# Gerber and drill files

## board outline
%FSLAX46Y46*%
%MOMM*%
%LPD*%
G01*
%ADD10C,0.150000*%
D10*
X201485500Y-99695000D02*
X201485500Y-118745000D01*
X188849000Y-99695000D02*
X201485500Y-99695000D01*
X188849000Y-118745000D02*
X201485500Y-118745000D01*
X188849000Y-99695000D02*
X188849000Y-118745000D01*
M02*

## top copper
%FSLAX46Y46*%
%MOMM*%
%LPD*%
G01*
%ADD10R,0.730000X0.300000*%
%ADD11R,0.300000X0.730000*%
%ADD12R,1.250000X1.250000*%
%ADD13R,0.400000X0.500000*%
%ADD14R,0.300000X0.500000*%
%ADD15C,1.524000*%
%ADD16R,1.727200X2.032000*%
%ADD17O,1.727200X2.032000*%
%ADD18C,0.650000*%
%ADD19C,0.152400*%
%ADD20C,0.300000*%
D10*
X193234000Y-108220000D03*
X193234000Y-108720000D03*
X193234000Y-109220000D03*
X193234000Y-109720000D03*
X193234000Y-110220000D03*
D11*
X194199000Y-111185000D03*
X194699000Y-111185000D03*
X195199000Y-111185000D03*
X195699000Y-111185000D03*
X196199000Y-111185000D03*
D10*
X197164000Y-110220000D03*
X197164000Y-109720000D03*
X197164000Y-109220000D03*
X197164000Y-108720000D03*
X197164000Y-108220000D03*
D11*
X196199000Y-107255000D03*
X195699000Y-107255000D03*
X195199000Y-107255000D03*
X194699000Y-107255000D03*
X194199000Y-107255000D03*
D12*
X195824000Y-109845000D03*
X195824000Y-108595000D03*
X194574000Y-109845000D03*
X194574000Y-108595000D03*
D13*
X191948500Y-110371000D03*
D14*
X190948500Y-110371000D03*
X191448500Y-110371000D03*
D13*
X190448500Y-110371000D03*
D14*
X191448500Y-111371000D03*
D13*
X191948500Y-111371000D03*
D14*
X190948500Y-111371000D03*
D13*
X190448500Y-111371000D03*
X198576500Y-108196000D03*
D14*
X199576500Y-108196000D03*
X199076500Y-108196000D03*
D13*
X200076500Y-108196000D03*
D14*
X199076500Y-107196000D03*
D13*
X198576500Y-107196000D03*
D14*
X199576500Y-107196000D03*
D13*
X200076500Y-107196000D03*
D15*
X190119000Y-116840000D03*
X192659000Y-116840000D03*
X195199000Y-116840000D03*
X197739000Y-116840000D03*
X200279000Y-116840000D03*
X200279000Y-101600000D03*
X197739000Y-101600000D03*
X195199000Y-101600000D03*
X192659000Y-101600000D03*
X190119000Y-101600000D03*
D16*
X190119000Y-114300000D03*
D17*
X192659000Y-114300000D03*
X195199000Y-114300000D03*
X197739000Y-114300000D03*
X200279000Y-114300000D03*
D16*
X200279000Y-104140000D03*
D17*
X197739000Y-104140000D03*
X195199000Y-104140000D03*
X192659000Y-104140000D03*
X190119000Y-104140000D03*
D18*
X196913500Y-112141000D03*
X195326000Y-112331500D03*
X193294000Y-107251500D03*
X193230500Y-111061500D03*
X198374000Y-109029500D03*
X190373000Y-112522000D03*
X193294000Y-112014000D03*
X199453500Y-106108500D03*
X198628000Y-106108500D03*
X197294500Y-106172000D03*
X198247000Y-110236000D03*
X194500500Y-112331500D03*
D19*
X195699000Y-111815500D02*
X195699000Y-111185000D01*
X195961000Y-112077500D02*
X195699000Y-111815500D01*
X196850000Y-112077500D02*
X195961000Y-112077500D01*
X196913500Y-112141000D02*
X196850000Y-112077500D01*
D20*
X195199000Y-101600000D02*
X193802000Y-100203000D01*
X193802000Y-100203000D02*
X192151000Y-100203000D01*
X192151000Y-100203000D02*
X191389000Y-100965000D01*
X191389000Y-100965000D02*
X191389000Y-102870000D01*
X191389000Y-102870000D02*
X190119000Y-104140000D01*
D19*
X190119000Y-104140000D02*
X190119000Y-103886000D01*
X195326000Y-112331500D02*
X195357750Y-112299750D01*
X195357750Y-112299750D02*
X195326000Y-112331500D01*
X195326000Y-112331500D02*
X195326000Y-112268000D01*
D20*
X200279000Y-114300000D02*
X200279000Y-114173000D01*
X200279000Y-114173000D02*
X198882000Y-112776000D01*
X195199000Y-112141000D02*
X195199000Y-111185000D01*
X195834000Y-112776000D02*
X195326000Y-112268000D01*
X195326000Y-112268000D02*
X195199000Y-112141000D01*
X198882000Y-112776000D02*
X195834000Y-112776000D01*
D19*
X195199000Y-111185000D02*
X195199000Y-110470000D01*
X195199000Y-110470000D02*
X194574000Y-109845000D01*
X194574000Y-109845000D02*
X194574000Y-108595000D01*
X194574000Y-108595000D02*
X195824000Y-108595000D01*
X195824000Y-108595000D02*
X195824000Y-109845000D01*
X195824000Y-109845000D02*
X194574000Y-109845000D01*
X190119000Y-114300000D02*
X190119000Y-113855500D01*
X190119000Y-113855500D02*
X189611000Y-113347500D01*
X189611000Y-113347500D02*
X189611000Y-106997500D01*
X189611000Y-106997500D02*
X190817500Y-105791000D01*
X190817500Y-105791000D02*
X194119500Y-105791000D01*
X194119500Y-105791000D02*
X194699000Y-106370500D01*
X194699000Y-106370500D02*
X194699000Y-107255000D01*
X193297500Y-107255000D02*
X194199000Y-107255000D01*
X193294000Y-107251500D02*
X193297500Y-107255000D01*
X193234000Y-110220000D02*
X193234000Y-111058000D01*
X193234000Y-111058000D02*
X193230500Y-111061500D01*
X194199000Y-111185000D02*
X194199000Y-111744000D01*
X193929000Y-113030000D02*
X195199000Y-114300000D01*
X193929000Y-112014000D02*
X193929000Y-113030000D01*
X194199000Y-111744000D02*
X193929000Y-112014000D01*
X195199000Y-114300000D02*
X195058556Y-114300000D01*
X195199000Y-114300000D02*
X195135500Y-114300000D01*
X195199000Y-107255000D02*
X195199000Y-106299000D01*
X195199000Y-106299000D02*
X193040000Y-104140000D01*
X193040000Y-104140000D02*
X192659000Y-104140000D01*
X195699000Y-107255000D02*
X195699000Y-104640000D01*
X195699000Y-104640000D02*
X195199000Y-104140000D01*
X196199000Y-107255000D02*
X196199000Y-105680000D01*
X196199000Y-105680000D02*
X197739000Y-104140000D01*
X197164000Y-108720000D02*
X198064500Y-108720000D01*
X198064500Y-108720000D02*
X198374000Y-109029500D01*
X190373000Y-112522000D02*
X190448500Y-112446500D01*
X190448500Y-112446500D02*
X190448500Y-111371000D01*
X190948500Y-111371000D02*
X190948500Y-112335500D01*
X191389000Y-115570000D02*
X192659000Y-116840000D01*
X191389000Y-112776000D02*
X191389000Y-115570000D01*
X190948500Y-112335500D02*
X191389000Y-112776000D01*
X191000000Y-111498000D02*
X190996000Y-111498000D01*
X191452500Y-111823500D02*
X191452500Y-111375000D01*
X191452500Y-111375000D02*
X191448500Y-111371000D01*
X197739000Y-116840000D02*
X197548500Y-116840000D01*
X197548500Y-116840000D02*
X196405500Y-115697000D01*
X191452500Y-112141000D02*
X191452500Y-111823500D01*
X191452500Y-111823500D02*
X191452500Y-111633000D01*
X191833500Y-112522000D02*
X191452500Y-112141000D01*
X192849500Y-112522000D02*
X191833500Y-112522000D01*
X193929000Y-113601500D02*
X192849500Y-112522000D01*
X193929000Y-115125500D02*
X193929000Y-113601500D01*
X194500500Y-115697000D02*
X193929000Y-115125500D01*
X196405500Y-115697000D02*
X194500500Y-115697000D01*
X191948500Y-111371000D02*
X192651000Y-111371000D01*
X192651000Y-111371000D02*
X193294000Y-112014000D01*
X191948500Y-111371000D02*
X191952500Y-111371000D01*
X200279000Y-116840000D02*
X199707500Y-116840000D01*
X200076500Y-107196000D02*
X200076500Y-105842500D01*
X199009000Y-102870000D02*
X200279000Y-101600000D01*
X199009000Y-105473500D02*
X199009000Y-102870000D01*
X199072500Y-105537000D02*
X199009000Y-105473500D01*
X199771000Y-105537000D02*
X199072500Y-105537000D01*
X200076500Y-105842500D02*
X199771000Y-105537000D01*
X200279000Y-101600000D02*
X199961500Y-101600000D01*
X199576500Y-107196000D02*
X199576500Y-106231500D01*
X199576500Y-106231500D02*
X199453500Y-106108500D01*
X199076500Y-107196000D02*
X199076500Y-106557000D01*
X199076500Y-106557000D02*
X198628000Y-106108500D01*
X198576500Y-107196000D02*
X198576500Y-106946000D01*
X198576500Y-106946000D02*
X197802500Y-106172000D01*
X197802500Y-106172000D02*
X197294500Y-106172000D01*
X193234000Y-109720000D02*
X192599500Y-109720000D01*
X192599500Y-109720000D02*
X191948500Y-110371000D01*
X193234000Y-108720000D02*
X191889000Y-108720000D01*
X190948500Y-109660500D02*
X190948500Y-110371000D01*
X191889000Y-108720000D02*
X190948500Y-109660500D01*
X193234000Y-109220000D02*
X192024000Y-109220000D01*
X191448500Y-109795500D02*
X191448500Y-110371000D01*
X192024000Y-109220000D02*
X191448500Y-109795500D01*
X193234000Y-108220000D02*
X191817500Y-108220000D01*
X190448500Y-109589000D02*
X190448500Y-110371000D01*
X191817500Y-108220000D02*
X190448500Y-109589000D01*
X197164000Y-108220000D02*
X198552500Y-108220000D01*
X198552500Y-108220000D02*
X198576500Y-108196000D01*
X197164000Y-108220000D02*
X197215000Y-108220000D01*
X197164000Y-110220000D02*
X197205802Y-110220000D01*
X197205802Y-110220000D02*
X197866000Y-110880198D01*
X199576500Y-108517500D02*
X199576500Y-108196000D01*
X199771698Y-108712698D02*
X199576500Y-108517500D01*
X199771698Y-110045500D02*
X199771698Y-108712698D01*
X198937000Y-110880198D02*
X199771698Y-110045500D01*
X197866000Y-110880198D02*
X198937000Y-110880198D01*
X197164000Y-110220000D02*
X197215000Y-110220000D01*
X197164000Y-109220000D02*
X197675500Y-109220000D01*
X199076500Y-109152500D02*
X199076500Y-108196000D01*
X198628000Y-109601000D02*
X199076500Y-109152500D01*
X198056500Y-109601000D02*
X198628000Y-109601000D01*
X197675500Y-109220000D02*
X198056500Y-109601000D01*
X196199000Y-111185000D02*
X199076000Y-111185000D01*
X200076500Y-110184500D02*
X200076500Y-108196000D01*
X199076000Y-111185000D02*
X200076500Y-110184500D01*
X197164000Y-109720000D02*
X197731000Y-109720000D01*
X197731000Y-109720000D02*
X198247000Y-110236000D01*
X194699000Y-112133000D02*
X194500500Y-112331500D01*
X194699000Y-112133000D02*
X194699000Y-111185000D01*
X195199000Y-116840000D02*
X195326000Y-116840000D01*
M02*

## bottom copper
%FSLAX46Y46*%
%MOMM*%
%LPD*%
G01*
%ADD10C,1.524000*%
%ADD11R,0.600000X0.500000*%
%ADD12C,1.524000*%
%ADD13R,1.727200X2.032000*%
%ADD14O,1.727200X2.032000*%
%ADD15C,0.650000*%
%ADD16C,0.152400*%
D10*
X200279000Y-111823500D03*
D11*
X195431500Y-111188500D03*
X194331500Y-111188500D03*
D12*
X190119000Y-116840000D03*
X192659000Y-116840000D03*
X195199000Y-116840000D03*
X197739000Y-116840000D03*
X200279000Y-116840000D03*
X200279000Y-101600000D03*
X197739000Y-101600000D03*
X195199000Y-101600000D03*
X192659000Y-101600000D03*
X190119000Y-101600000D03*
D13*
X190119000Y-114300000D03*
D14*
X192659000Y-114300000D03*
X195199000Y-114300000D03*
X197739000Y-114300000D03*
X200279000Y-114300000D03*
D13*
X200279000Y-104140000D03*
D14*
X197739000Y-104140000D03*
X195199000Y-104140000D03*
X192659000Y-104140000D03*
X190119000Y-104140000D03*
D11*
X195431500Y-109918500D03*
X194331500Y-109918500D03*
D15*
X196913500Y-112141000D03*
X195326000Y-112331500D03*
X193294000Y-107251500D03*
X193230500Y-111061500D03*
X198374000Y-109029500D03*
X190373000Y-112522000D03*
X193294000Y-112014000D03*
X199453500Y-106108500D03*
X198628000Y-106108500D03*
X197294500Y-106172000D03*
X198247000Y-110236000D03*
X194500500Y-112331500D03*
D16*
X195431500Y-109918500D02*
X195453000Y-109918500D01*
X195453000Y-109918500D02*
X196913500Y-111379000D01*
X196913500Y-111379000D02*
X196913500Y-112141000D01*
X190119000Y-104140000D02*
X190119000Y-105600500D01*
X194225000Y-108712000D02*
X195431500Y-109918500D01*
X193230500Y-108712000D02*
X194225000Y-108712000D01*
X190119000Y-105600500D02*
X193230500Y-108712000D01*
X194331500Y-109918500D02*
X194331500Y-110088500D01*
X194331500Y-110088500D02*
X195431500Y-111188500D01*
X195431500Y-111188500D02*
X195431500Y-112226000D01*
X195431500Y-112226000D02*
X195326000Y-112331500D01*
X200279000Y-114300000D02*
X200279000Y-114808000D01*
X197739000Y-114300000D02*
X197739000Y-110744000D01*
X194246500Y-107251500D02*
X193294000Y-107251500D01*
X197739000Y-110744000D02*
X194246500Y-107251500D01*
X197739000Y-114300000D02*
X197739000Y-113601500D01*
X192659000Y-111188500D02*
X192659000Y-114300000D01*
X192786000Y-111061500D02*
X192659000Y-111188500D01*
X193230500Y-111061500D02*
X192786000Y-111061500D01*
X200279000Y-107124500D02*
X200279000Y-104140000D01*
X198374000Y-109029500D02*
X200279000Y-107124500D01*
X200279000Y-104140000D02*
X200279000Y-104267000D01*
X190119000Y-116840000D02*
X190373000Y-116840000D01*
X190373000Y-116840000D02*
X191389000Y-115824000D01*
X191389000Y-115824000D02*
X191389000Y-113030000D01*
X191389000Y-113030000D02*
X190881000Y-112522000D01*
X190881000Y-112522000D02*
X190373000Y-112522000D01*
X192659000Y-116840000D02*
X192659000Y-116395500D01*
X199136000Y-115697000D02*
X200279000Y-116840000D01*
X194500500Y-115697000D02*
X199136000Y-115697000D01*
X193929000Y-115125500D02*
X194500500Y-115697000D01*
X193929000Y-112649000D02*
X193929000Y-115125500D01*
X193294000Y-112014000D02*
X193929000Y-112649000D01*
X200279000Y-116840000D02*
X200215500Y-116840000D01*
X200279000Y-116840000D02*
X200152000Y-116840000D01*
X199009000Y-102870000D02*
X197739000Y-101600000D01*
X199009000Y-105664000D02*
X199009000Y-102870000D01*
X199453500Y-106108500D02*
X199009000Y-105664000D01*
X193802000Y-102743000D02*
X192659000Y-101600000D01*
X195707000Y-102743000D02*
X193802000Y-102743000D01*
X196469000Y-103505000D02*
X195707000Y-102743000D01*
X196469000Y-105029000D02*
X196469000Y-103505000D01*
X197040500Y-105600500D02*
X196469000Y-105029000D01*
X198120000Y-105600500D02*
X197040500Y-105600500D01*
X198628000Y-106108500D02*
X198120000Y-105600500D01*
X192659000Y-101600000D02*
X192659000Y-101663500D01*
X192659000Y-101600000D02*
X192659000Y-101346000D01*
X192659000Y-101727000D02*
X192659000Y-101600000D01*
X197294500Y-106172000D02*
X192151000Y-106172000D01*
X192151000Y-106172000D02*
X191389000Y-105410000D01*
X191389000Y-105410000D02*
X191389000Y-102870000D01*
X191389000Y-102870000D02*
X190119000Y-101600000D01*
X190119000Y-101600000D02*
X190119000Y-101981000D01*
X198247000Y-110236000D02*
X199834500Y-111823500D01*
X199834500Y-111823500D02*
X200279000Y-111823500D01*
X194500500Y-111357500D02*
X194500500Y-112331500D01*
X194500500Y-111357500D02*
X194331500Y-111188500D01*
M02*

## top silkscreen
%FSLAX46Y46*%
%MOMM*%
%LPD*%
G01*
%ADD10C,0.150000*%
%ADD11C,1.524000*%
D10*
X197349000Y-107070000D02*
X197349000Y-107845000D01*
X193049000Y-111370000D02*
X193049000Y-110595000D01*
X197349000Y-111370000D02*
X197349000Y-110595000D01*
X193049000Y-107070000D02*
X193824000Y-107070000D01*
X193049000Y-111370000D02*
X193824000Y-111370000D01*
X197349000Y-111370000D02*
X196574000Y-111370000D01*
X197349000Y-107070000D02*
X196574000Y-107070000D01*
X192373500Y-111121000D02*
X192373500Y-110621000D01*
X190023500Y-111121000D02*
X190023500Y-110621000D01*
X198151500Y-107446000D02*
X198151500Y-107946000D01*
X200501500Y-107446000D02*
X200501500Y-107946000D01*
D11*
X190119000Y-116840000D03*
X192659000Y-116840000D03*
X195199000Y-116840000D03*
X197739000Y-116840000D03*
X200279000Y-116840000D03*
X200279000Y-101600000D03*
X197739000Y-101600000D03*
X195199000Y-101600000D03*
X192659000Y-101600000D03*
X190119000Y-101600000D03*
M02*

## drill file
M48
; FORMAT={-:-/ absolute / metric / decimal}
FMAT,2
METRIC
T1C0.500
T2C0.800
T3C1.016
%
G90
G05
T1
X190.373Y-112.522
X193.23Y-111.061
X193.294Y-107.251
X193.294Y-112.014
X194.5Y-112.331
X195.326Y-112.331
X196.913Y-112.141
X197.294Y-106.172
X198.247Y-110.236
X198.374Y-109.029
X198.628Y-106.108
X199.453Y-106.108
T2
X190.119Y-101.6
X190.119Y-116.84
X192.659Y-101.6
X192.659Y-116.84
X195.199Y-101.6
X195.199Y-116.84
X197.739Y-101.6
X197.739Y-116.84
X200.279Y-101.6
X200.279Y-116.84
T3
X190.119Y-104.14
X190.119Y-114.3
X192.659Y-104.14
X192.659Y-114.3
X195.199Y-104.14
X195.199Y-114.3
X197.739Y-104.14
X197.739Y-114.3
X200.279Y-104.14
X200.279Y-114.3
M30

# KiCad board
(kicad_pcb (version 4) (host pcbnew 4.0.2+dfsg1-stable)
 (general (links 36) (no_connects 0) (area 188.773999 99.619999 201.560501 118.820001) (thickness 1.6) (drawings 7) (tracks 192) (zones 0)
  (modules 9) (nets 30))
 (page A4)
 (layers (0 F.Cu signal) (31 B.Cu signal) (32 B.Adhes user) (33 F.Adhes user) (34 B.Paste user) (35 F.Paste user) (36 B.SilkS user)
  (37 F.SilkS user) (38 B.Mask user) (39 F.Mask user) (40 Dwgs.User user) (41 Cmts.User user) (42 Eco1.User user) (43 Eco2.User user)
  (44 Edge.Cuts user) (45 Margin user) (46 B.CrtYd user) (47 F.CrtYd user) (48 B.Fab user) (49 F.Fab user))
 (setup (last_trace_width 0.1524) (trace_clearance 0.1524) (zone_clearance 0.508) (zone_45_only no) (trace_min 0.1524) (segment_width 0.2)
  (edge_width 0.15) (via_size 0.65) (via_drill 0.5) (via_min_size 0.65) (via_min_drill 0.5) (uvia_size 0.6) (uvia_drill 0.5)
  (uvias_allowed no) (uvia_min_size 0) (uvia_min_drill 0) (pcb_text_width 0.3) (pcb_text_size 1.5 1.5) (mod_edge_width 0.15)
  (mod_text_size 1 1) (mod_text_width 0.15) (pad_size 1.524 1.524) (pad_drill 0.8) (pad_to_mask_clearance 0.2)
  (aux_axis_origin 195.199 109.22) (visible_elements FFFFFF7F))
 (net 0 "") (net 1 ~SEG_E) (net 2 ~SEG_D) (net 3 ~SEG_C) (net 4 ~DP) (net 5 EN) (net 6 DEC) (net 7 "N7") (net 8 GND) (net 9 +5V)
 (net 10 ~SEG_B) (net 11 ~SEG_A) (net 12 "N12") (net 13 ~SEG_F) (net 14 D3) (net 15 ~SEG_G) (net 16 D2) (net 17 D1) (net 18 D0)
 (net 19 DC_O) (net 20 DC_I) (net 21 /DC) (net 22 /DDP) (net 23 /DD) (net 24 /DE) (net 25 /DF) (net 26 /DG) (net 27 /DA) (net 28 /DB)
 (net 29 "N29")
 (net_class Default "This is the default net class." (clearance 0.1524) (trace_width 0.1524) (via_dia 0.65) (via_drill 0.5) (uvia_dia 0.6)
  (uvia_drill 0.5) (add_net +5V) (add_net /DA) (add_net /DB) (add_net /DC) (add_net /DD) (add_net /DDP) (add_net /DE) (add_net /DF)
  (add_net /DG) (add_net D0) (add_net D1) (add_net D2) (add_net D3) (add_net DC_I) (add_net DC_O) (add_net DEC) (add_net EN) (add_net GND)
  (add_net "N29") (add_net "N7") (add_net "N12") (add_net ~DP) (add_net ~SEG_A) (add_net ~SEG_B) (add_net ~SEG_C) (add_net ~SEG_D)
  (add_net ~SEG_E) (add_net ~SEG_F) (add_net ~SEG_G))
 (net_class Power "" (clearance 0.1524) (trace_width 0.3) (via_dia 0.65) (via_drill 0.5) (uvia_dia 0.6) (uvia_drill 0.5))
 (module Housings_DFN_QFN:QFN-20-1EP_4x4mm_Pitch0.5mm (layer F.Cu) (at 195.199 109.22)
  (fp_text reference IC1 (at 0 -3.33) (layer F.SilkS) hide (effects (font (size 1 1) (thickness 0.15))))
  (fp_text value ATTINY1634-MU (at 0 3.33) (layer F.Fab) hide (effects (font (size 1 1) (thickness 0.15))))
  (fp_line (start 2.15 -2.15) (end 2.15 -1.375) (layer F.SilkS) (width 0.15))
  (fp_line (start -2.15 2.15) (end -2.15 1.375) (layer F.SilkS) (width 0.15))
  (fp_line (start 2.15 2.15) (end 2.15 1.375) (layer F.SilkS) (width 0.15))
  (fp_line (start -2.15 -2.15) (end -1.375 -2.15) (layer F.SilkS) (width 0.15))
  (fp_line (start -2.15 2.15) (end -1.375 2.15) (layer F.SilkS) (width 0.15))
  (fp_line (start 2.15 2.15) (end 1.375 2.15) (layer F.SilkS) (width 0.15))
  (fp_line (start 2.15 -2.15) (end 1.375 -2.15) (layer F.SilkS) (width 0.15))
  (pad 1 smd rect (at -1.965 -1) (size 0.73 0.3) (layers F.Cu F.Paste F.Mask) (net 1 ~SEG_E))
  (pad 2 smd rect (at -1.965 -0.5) (size 0.73 0.3) (layers F.Cu F.Paste F.Mask) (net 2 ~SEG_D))
  (pad 3 smd rect (at -1.965 0) (size 0.73 0.3) (layers F.Cu F.Paste F.Mask) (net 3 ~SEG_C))
  (pad 4 smd rect (at -1.965 0.5) (size 0.73 0.3) (layers F.Cu F.Paste F.Mask) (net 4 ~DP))
  (pad 5 smd rect (at -1.965 1) (size 0.73 0.3) (layers F.Cu F.Paste F.Mask) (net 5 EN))
  (pad 6 smd rect (at -1 1.965 90) (size 0.73 0.3) (layers F.Cu F.Paste F.Mask) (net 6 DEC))
  (pad 7 smd rect (at -0.5 1.965 90) (size 0.73 0.3) (layers F.Cu F.Paste F.Mask) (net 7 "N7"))
  (pad 8 smd rect (at 0 1.965 90) (size 0.73 0.3) (layers F.Cu F.Paste F.Mask) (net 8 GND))
  (pad 9 smd rect (at 0.5 1.965 90) (size 0.73 0.3) (layers F.Cu F.Paste F.Mask) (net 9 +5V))
  (pad 10 smd rect (at 1 1.965 90) (size 0.73 0.3) (layers F.Cu F.Paste F.Mask) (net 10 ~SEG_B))
  (pad 11 smd rect (at 1.965 1) (size 0.73 0.3) (layers F.Cu F.Paste F.Mask) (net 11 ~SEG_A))
  (pad 12 smd rect (at 1.965 0.5) (size 0.73 0.3) (layers F.Cu F.Paste F.Mask) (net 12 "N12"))
  (pad 13 smd rect (at 1.965 0) (size 0.73 0.3) (layers F.Cu F.Paste F.Mask) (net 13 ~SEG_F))
  (pad 14 smd rect (at 1.965 -0.5) (size 0.73 0.3) (layers F.Cu F.Paste F.Mask) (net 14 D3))
  (pad 15 smd rect (at 1.965 -1) (size 0.73 0.3) (layers F.Cu F.Paste F.Mask) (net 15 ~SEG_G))
  (pad 16 smd rect (at 1 -1.965 90) (size 0.73 0.3) (layers F.Cu F.Paste F.Mask) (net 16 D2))
  (pad 17 smd rect (at 0.5 -1.965 90) (size 0.73 0.3) (layers F.Cu F.Paste F.Mask) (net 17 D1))
  (pad 18 smd rect (at 0 -1.965 90) (size 0.73 0.3) (layers F.Cu F.Paste F.Mask) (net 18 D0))
  (pad 19 smd rect (at -0.5 -1.965 90) (size 0.73 0.3) (layers F.Cu F.Paste F.Mask) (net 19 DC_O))
  (pad 20 smd rect (at -1 -1.965 90) (size 0.73 0.3) (layers F.Cu F.Paste F.Mask) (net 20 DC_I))
  (pad 21 smd rect (at 0.625 0.625) (size 1.25 1.25) (layers F.Cu F.Paste F.Mask) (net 8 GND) (solder_paste_margin_ratio -0.2))
  (pad 21 smd rect (at 0.625 -0.625) (size 1.25 1.25) (layers F.Cu F.Paste F.Mask) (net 8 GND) (solder_paste_margin_ratio -0.2))
  (pad 21 smd rect (at -0.625 0.625) (size 1.25 1.25) (layers F.Cu F.Paste F.Mask) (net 8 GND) (solder_paste_margin_ratio -0.2))
  (pad 21 smd rect (at -0.625 -0.625) (size 1.25 1.25) (layers F.Cu F.Paste F.Mask) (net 8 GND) (solder_paste_margin_ratio -0.2)))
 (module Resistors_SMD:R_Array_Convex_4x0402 (layer F.Cu) (at 191.1985 110.871 270)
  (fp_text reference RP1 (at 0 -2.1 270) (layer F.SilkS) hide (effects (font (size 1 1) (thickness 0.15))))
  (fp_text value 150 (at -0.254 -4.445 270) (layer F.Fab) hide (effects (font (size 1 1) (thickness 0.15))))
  (fp_line (start 0.25 -1.175) (end -0.25 -1.175) (layer F.SilkS) (width 0.15))
  (fp_line (start 0.25 1.175) (end -0.25 1.175) (layer F.SilkS) (width 0.15))
  (pad 1 smd rect (at -0.5 -0.75 270) (size 0.5 0.4) (layers F.Cu F.Paste F.Mask) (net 4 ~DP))
  (pad 3 smd rect (at -0.5 0.25 270) (size 0.5 0.3) (layers F.Cu F.Paste F.Mask) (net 2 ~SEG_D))
  (pad 2 smd rect (at -0.5 -0.25 270) (size 0.5 0.3) (layers F.Cu F.Paste F.Mask) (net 3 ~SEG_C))
  (pad 4 smd rect (at -0.5 0.75 270) (size 0.5 0.4) (layers F.Cu F.Paste F.Mask) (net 1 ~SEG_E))
  (pad 7 smd rect (at 0.5 -0.25 270) (size 0.5 0.3) (layers F.Cu F.Paste F.Mask) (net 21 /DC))
  (pad 8 smd rect (at 0.5 -0.75 270) (size 0.5 0.4) (layers F.Cu F.Paste F.Mask) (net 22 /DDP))
  (pad 6 smd rect (at 0.5 0.25 270) (size 0.5 0.3) (layers F.Cu F.Paste F.Mask) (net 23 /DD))
  (pad 5 smd rect (at 0.5 0.75 270) (size 0.5 0.4) (layers F.Cu F.Paste F.Mask) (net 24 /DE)))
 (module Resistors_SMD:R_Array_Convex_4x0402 (layer F.Cu) (at 199.3265 107.696 90)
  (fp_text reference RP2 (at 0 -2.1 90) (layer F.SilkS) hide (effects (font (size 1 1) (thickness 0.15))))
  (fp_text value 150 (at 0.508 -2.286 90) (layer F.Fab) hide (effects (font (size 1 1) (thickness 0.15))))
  (fp_line (start 0.25 -1.175) (end -0.25 -1.175) (layer F.SilkS) (width 0.15))
  (fp_line (start 0.25 1.175) (end -0.25 1.175) (layer F.SilkS) (width 0.15))
  (pad 1 smd rect (at -0.5 -0.75 90) (size 0.5 0.4) (layers F.Cu F.Paste F.Mask) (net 15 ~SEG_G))
  (pad 3 smd rect (at -0.5 0.25 90) (size 0.5 0.3) (layers F.Cu F.Paste F.Mask) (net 11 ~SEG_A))
  (pad 2 smd rect (at -0.5 -0.25 90) (size 0.5 0.3) (layers F.Cu F.Paste F.Mask) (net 13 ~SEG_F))
  (pad 4 smd rect (at -0.5 0.75 90) (size 0.5 0.4) (layers F.Cu F.Paste F.Mask) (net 10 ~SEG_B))
  (pad 7 smd rect (at 0.5 -0.25 90) (size 0.5 0.3) (layers F.Cu F.Paste F.Mask) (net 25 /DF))
  (pad 8 smd rect (at 0.5 -0.75 90) (size 0.5 0.4) (layers F.Cu F.Paste F.Mask) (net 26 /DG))
  (pad 6 smd rect (at 0.5 0.25 90) (size 0.5 0.3) (layers F.Cu F.Paste F.Mask) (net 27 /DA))
  (pad 5 smd rect (at 0.5 0.75 90) (size 0.5 0.4) (layers F.Cu F.Paste F.Mask) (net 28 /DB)))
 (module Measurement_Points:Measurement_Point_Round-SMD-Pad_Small (layer B.Cu) (at 200.279 111.8235)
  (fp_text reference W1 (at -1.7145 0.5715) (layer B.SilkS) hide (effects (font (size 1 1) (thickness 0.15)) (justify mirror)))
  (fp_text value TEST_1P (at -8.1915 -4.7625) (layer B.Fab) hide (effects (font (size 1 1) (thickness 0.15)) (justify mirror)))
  (pad 1 smd circle (at 0 0) (size 1.524 1.524) (layers B.Cu B.Paste B.Mask) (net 12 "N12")))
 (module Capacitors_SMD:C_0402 (layer B.Cu) (at 194.8815 111.1885 180)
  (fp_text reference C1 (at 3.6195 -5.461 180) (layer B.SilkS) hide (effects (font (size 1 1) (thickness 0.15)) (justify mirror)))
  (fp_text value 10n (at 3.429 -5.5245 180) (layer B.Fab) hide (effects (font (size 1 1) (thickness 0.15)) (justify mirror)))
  (pad 1 smd rect (at -0.55 0 180) (size 0.6 0.5) (layers B.Cu B.Paste B.Mask) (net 8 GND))
  (pad 2 smd rect (at 0.55 0 180) (size 0.6 0.5) (layers B.Cu B.Paste B.Mask) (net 7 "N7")))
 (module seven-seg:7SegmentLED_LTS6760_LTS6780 (layer F.Cu) (at 195.199 109.22)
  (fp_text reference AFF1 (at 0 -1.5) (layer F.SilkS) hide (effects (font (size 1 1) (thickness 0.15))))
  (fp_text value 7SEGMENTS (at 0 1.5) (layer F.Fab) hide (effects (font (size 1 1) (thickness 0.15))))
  (pad 1 thru_hole circle (at -5.08 7.62) (size 1.524 1.524) (drill 0.8) (layers *.Cu *.Mask F.SilkS) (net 24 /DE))
  (pad 2 thru_hole circle (at -2.54 7.62) (size 1.524 1.524) (drill 0.8) (layers *.Cu *.Mask F.SilkS) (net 23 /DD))
  (pad 3 thru_hole circle (at 0 7.62) (size 1.524 1.524) (drill 0.8) (layers *.Cu *.Mask F.SilkS) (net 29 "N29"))
  (pad 4 thru_hole circle (at 2.54 7.62) (size 1.524 1.524) (drill 0.8) (layers *.Cu *.Mask F.SilkS) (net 21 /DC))
  (pad 5 thru_hole circle (at 5.08 7.62) (size 1.524 1.524) (drill 0.8) (layers *.Cu *.Mask F.SilkS) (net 22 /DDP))
  (pad 6 thru_hole circle (at 5.08 -7.62) (size 1.524 1.524) (drill 0.8) (layers *.Cu *.Mask F.SilkS) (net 28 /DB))
  (pad 7 thru_hole circle (at 2.54 -7.62) (size 1.524 1.524) (drill 0.8) (layers *.Cu *.Mask F.SilkS) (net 27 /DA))
  (pad 8 thru_hole circle (at 0 -7.62) (size 1.524 1.524) (drill 0.8) (layers *.Cu *.Mask F.SilkS) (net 9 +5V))
  (pad 9 thru_hole circle (at -2.54 -7.62) (size 1.524 1.524) (drill 0.8) (layers *.Cu *.Mask F.SilkS) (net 25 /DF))
  (pad 10 thru_hole circle (at -5.08 -7.62) (size 1.524 1.524) (drill 0.8) (layers *.Cu *.Mask F.SilkS) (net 26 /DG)))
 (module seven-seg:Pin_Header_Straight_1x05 (layer B.Cu) (at 190.119 114.3 270)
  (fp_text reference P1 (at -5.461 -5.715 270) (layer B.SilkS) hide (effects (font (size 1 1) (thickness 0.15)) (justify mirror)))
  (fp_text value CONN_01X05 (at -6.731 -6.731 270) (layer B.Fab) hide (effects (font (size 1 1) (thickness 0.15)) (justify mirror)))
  (pad 1 thru_hole rect (at 0 0 270) (size 2.032 1.7272) (drill 1.016) (layers *.Cu *.Mask B.SilkS) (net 19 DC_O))
  (pad 2 thru_hole oval (at 0 -2.54 270) (size 2.032 1.7272) (drill 1.016) (layers *.Cu *.Mask B.SilkS) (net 5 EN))
  (pad 3 thru_hole oval (at 0 -5.08 270) (size 2.032 1.7272) (drill 1.016) (layers *.Cu *.Mask B.SilkS) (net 6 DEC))
  (pad 4 thru_hole oval (at 0 -7.62 270) (size 2.032 1.7272) (drill 1.016) (layers *.Cu *.Mask B.SilkS) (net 20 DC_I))
  (pad 5 thru_hole oval (at 0 -10.16 270) (size 2.032 1.7272) (drill 1.016) (layers *.Cu *.Mask B.SilkS) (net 8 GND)))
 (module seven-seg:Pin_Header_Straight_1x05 (layer B.Cu) (at 200.279 104.14 90)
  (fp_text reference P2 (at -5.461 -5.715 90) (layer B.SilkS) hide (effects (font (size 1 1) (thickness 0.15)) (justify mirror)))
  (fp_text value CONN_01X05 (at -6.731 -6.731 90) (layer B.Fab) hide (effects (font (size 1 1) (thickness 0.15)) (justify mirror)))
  (pad 1 thru_hole rect (at 0 0 90) (size 2.032 1.7272) (drill 1.016) (layers *.Cu *.Mask B.SilkS) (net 14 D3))
  (pad 2 thru_hole oval (at 0 -2.54 90) (size 2.032 1.7272) (drill 1.016) (layers *.Cu *.Mask B.SilkS) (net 16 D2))
  (pad 3 thru_hole oval (at 0 -5.08 90) (size 2.032 1.7272) (drill 1.016) (layers *.Cu *.Mask B.SilkS) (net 17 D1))
  (pad 4 thru_hole oval (at 0 -7.62 90) (size 2.032 1.7272) (drill 1.016) (layers *.Cu *.Mask B.SilkS) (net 18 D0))
  (pad 5 thru_hole oval (at 0 -10.16 90) (size 2.032 1.7272) (drill 1.016) (layers *.Cu *.Mask B.SilkS) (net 9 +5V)))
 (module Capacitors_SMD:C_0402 (layer B.Cu) (at 194.8815 109.9185 180)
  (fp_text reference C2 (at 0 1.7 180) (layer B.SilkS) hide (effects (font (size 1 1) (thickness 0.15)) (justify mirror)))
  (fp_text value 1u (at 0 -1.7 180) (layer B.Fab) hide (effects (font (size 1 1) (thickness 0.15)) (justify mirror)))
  (pad 1 smd rect (at -0.55 0 180) (size 0.6 0.5) (layers B.Cu B.Paste B.Mask) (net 9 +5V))
  (pad 2 smd rect (at 0.55 0 180) (size 0.6 0.5) (layers B.Cu B.Paste B.Mask) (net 8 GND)))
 (gr_line (start 201.4855 99.695) (end 201.4855 118.745) (angle 90) (layer Edge.Cuts) (width 0.15))
 (gr_line (start 188.849 99.695) (end 201.4855 99.695) (angle 90) (layer Edge.Cuts) (width 0.15))
 (gr_line (start 188.849 118.745) (end 201.4855 118.745) (angle 90) (layer Edge.Cuts) (width 0.15))
 (gr_line (start 188.849 99.695) (end 188.849 118.745) (angle 90) (layer Edge.Cuts) (width 0.15))
 (segment (start 195.4315 109.9185) (end 195.453 109.9185) (width 0.1524) (layer B.Cu) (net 9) (status C00000))
 (segment (start 195.453 109.9185) (end 196.9135 111.379) (width 0.1524) (layer B.Cu) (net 9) (status 400000))
 (segment (start 195.699 111.8155) (end 195.699 111.185) (width 0.1524) (layer F.Cu) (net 9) (status 800000))
 (segment (start 195.961 112.0775) (end 195.699 111.8155) (width 0.1524) (layer F.Cu) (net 9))
 (segment (start 196.85 112.0775) (end 195.961 112.0775) (width 0.1524) (layer F.Cu) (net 9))
 (segment (start 196.9135 112.141) (end 196.85 112.0775) (width 0.1524) (layer F.Cu) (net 9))
 (via (at 196.9135 112.141) (size 0.65) (drill 0.5) (layers F.Cu B.Cu) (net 9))
 (segment (start 196.9135 111.379) (end 196.9135 112.141) (width 0.1524) (layer B.Cu) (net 9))
 (segment (start 190.119 104.14) (end 190.119 105.6005) (width 0.1524) (layer B.Cu) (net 9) (status 400000))
 (segment (start 194.225 108.712) (end 195.4315 109.9185) (width 0.1524) (layer B.Cu) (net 9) (status 800000))
 (segment (start 193.2305 108.712) (end 194.225 108.712) (width 0.1524) (layer B.Cu) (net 9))
 (segment (start 190.119 105.6005) (end 193.2305 108.712) (width 0.1524) (layer B.Cu) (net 9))
 (segment (start 195.199 101.6) (end 193.802 100.203) (width 0.3) (layer F.Cu) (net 9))
 (segment (start 193.802 100.203) (end 192.151 100.203) (width 0.3) (layer F.Cu) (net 9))
 (segment (start 192.151 100.203) (end 191.389 100.965) (width 0.3) (layer F.Cu) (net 9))
 (segment (start 191.389 100.965) (end 191.389 102.87) (width 0.3) (layer F.Cu) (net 9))
 (segment (start 191.389 102.87) (end 190.119 104.14) (width 0.3) (layer F.Cu) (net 9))
 (segment (start 190.119 104.14) (end 190.119 103.886) (width 0.1524) (layer F.Cu) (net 9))
 (segment (start 194.3315 109.9185) (end 194.3315 110.0885) (width 0.1524) (layer B.Cu) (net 8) (status C00000))
 (segment (start 194.3315 110.0885) (end 195.4315 111.1885) (width 0.1524) (layer B.Cu) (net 8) (status C00000))
 (segment (start 195.4315 111.1885) (end 195.4315 112.226) (width 0.1524) (layer B.Cu) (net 8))
 (via (at 195.326 112.3315) (size 0.65) (drill 0.5) (layers F.Cu B.Cu) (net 8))
 (segment (start 195.4315 112.226) (end 195.326 112.3315) (width 0.1524) (layer B.Cu) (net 8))
 (segment (start 195.326 112.3315) (end 195.35775 112.29975) (width 0.1524) (layer F.Cu) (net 8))
 (segment (start 195.35775 112.29975) (end 195.326 112.3315) (width 0.1524) (layer F.Cu) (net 8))
 (segment (start 195.326 112.3315) (end 195.326 112.268) (width 0.1524) (layer F.Cu) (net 8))
 (segment (start 200.279 114.3) (end 200.279 114.173) (width 0.3) (layer F.Cu) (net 8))
 (segment (start 200.279 114.173) (end 198.882 112.776) (width 0.3) (layer F.Cu) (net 8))
 (segment (start 195.199 112.141) (end 195.199 111.185) (width 0.3) (layer F.Cu) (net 8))
 (segment (start 195.834 112.776) (end 195.326 112.268) (width 0.3) (layer F.Cu) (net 8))
 (segment (start 195.326 112.268) (end 195.199 112.141) (width 0.3) (layer F.Cu) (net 8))
 (segment (start 198.882 112.776) (end 195.834 112.776) (width 0.3) (layer F.Cu) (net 8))
 (segment (start 200.279 114.3) (end 200.279 114.808) (width 0.1524) (layer B.Cu) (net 8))
 (segment (start 195.199 111.185) (end 195.199 110.47) (width 0.1524) (layer F.Cu) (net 8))
 (segment (start 195.199 110.47) (end 194.574 109.845) (width 0.1524) (layer F.Cu) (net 8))
 (segment (start 194.574 109.845) (end 194.574 108.595) (width 0.1524) (layer F.Cu) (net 8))
 (segment (start 194.574 108.595) (end 195.824 108.595) (width 0.1524) (layer F.Cu) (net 8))
 (segment (start 195.824 108.595) (end 195.824 109.845) (width 0.1524) (layer F.Cu) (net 8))
 (segment (start 195.824 109.845) (end 194.574 109.845) (width 0.1524) (layer F.Cu) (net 8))
 (segment (start 190.119 114.3) (end 190.119 113.8555) (width 0.1524) (layer F.Cu) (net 19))
 (segment (start 190.119 113.8555) (end 189.611 113.3475) (width 0.1524) (layer F.Cu) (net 19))
 (segment (start 189.611 113.3475) (end 189.611 106.9975) (width 0.1524) (layer F.Cu) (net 19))
 (segment (start 189.611 106.9975) (end 190.8175 105.791) (width 0.1524) (layer F.Cu) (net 19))
 (segment (start 190.8175 105.791) (end 194.1195 105.791) (width 0.1524) (layer F.Cu) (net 19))
 (segment (start 194.1195 105.791) (end 194.699 106.3705) (width 0.1524) (layer F.Cu) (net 19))
 (segment (start 194.699 106.3705) (end 194.699 107.255) (width 0.1524) (layer F.Cu) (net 19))
 (segment (start 197.739 114.3) (end 197.739 110.744) (width 0.1524) (layer B.Cu) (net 20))
 (segment (start 193.2975 107.255) (end 194.199 107.255) (width 0.1524) (layer F.Cu) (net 20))
 (segment (start 193.294 107.2515) (end 193.2975 107.255) (width 0.1524) (layer F.Cu) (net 20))
 (via (at 193.294 107.2515) (size 0.65) (drill 0.5) (layers F.Cu B.Cu) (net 20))
 (segment (start 194.2465 107.2515) (end 193.294 107.2515) (width 0.1524) (layer B.Cu) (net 20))
 (segment (start 197.739 110.744) (end 194.2465 107.2515) (width 0.1524) (layer B.Cu) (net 20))
 (segment (start 197.739 114.3) (end 197.739 113.6015) (width 0.1524) (layer B.Cu) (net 20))
 (segment (start 193.234 110.22) (end 193.234 111.058) (width 0.1524) (layer F.Cu) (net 5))
 (segment (start 192.659 111.1885) (end 192.659 114.3) (width 0.1524) (layer B.Cu) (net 5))
 (segment (start 192.786 111.0615) (end 192.659 111.1885) (width 0.1524) (layer B.Cu) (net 5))
 (segment (start 193.2305 111.0615) (end 192.786 111.0615) (width 0.1524) (layer B.Cu) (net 5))
 (via (at 193.2305 111.0615) (size 0.65) (drill 0.5) (layers F.Cu B.Cu) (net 5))
 (segment (start 193.234 111.058) (end 193.2305 111.0615) (width 0.1524) (layer F.Cu) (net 5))
 (segment (start 194.199 111.185) (end 194.199 111.744) (width 0.1524) (layer F.Cu) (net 6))
 (segment (start 193.929 113.03) (end 195.199 114.3) (width 0.1524) (layer F.Cu) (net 6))
 (segment (start 193.929 112.014) (end 193.929 113.03) (width 0.1524) (layer F.Cu) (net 6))
 (segment (start 194.199 111.744) (end 193.929 112.014) (width 0.1524) (layer F.Cu) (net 6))
 (segment (start 195.199 114.3) (end 195.058556 114.3) (width 0.1524) (layer F.Cu) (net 6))
 (segment (start 195.199 114.3) (end 195.1355 114.3) (width 0.1524) (layer F.Cu) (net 6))
 (segment (start 195.199 107.255) (end 195.199 106.299) (width 0.1524) (layer F.Cu) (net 18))
 (segment (start 195.199 106.299) (end 193.04 104.14) (width 0.1524) (layer F.Cu) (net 18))
 (segment (start 193.04 104.14) (end 192.659 104.14) (width 0.1524) (layer F.Cu) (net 18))
 (segment (start 195.699 107.255) (end 195.699 104.64) (width 0.1524) (layer F.Cu) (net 17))
 (segment (start 195.699 104.64) (end 195.199 104.14) (width 0.1524) (layer F.Cu) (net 17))
 (segment (start 196.199 107.255) (end 196.199 105.68) (width 0.1524) (layer F.Cu) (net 16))
 (segment (start 196.199 105.68) (end 197.739 104.14) (width 0.1524) (layer F.Cu) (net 16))
 (segment (start 197.164 108.72) (end 198.0645 108.72) (width 0.1524) (layer F.Cu) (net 14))
 (segment (start 200.279 107.1245) (end 200.279 104.14) (width 0.1524) (layer B.Cu) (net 14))
 (segment (start 198.374 109.0295) (end 200.279 107.1245) (width 0.1524) (layer B.Cu) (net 14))
 (via (at 198.374 109.0295) (size 0.65) (drill 0.5) (layers F.Cu B.Cu) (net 14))
 (segment (start 198.0645 108.72) (end 198.374 109.0295) (width 0.1524) (layer F.Cu) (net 14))
 (segment (start 200.279 104.14) (end 200.279 104.267) (width 0.1524) (layer B.Cu) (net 14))
 (segment (start 190.119 116.84) (end 190.373 116.84) (width 0.1524) (layer B.Cu) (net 24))
 (segment (start 190.373 116.84) (end 191.389 115.824) (width 0.1524) (layer B.Cu) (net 24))
 (segment (start 191.389 115.824) (end 191.389 113.03) (width 0.1524) (layer B.Cu) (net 24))
 (segment (start 191.389 113.03) (end 190.881 112.522) (width 0.1524) (layer B.Cu) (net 24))
 (segment (start 190.881 112.522) (end 190.373 112.522) (width 0.1524) (layer B.Cu) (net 24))
 (via (at 190.373 112.522) (size 0.65) (drill 0.5) (layers F.Cu B.Cu) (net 24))
 (segment (start 190.373 112.522) (end 190.4485 112.4465) (width 0.1524) (layer F.Cu) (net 24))
 (segment (start 190.4485 112.4465) (end 190.4485 111.371) (width 0.1524) (layer F.Cu) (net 24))
 (segment (start 190.9485 111.371) (end 190.9485 112.3355) (width 0.1524) (layer F.Cu) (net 23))
 (segment (start 191.389 115.57) (end 192.659 116.84) (width 0.1524) (layer F.Cu) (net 23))
 (segment (start 191.389 112.776) (end 191.389 115.57) (width 0.1524) (layer F.Cu) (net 23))
 (segment (start 190.9485 112.3355) (end 191.389 112.776) (width 0.1524) (layer F.Cu) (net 23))
 (segment (start 192.659 116.84) (end 192.659 116.3955) (width 0.1524) (layer B.Cu) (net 23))
 (segment (start 191 111.498) (end 190.996 111.498) (width 0.1524) (layer F.Cu) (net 23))
 (segment (start 191.4525 111.8235) (end 191.4525 111.375) (width 0.1524) (layer F.Cu) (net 21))
 (segment (start 191.4525 111.375) (end 191.4485 111.371) (width 0.1524) (layer F.Cu) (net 21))
 (segment (start 197.739 116.84) (end 197.5485 116.84) (width 0.1524) (layer F.Cu) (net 21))
 (segment (start 197.5485 116.84) (end 196.4055 115.697) (width 0.1524) (layer F.Cu) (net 21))
 (segment (start 191.4525 112.141) (end 191.4525 111.8235) (width 0.1524) (layer F.Cu) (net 21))
 (segment (start 191.4525 111.8235) (end 191.4525 111.633) (width 0.1524) (layer F.Cu) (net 21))
 (segment (start 191.8335 112.522) (end 191.4525 112.141) (width 0.1524) (layer F.Cu) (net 21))
 (segment (start 192.8495 112.522) (end 191.8335 112.522) (width 0.1524) (layer F.Cu) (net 21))
 (segment (start 193.929 113.6015) (end 192.8495 112.522) (width 0.1524) (layer F.Cu) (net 21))
 (segment (start 193.929 115.1255) (end 193.929 113.6015) (width 0.1524) (layer F.Cu) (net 21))
 (segment (start 194.5005 115.697) (end 193.929 115.1255) (width 0.1524) (layer F.Cu) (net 21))
 (segment (start 196.4055 115.697) (end 194.5005 115.697) (width 0.1524) (layer F.Cu) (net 21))
 (segment (start 191.9485 111.371) (end 192.651 111.371) (width 0.1524) (layer F.Cu) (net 22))
 (segment (start 199.136 115.697) (end 200.279 116.84) (width 0.1524) (layer B.Cu) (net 22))
 (segment (start 194.5005 115.697) (end 199.136 115.697) (width 0.1524) (layer B.Cu) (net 22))
 (segment (start 193.929 115.1255) (end 194.5005 115.697) (width 0.1524) (layer B.Cu) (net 22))
 (segment (start 193.929 112.649) (end 193.929 115.1255) (width 0.1524) (layer B.Cu) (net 22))
 (segment (start 193.294 112.014) (end 193.929 112.649) (width 0.1524) (layer B.Cu) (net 22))
 (via (at 193.294 112.014) (size 0.65) (drill 0.5) (layers F.Cu B.Cu) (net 22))
 (segment (start 192.651 111.371) (end 193.294 112.014) (width 0.1524) (layer F.Cu) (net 22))
 (segment (start 191.9485 111.371) (end 191.9525 111.371) (width 0.1524) (layer F.Cu) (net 22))
 (segment (start 200.279 116.84) (end 199.7075 116.84) (width 0.1524) (layer F.Cu) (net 22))
 (segment (start 200.279 116.84) (end 200.2155 116.84) (width 0.1524) (layer B.Cu) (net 22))
 (segment (start 200.279 116.84) (end 200.152 116.84) (width 0.1524) (layer B.Cu) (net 22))
 (segment (start 200.0765 107.196) (end 200.0765 105.8425) (width 0.1524) (layer F.Cu) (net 28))
 (segment (start 199.009 102.87) (end 200.279 101.6) (width 0.1524) (layer F.Cu) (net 28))
 (segment (start 199.009 105.4735) (end 199.009 102.87) (width 0.1524) (layer F.Cu) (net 28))
 (segment (start 199.0725 105.537) (end 199.009 105.4735) (width 0.1524) (layer F.Cu) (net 28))
 (segment (start 199.771 105.537) (end 199.0725 105.537) (width 0.1524) (layer F.Cu) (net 28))
 (segment (start 200.0765 105.8425) (end 199.771 105.537) (width 0.1524) (layer F.Cu) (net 28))
 (segment (start 200.279 101.6) (end 199.9615 101.6) (width 0.1524) (layer F.Cu) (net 28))
 (segment (start 199.5765 107.196) (end 199.5765 106.2315) (width 0.1524) (layer F.Cu) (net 27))
 (segment (start 199.009 102.87) (end 197.739 101.6) (width 0.1524) (layer B.Cu) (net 27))
 (segment (start 199.009 105.664) (end 199.009 102.87) (width 0.1524) (layer B.Cu) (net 27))
 (segment (start 199.4535 106.1085) (end 199.009 105.664) (width 0.1524) (layer B.Cu) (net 27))
 (via (at 199.4535 106.1085) (size 0.65) (drill 0.5) (layers F.Cu B.Cu) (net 27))
 (segment (start 199.5765 106.2315) (end 199.4535 106.1085) (width 0.1524) (layer F.Cu) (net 27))
 (segment (start 199.0765 107.196) (end 199.0765 106.557) (width 0.1524) (layer F.Cu) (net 25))
 (segment (start 193.802 102.743) (end 192.659 101.6) (width 0.1524) (layer B.Cu) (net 25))
 (segment (start 195.707 102.743) (end 193.802 102.743) (width 0.1524) (layer B.Cu) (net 25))
 (segment (start 196.469 103.505) (end 195.707 102.743) (width 0.1524) (layer B.Cu) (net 25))
 (segment (start 196.469 105.029) (end 196.469 103.505) (width 0.1524) (layer B.Cu) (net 25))
 (segment (start 197.0405 105.6005) (end 196.469 105.029) (width 0.1524) (layer B.Cu) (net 25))
 (segment (start 198.12 105.6005) (end 197.0405 105.6005) (width 0.1524) (layer B.Cu) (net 25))
 (segment (start 198.628 106.1085) (end 198.12 105.6005) (width 0.1524) (layer B.Cu) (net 25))
 (via (at 198.628 106.1085) (size 0.65) (drill 0.5) (layers F.Cu B.Cu) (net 25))
 (segment (start 199.0765 106.557) (end 198.628 106.1085) (width 0.1524) (layer F.Cu) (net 25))
 (segment (start 192.659 101.6) (end 192.659 101.6635) (width 0.1524) (layer B.Cu) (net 25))
 (segment (start 192.659 101.6) (end 192.659 101.346) (width 0.1524) (layer B.Cu) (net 25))
 (segment (start 192.659 101.727) (end 192.659 101.6) (width 0.1524) (layer B.Cu) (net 25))
 (segment (start 198.5765 107.196) (end 198.5765 106.946) (width 0.1524) (layer F.Cu) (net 26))
 (segment (start 198.5765 106.946) (end 197.8025 106.172) (width 0.1524) (layer F.Cu) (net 26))
 (segment (start 197.8025 106.172) (end 197.2945 106.172) (width 0.1524) (layer F.Cu) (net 26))
 (via (at 197.2945 106.172) (size 0.65) (drill 0.5) (layers F.Cu B.Cu) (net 26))
 (segment (start 197.2945 106.172) (end 192.151 106.172) (width 0.1524) (layer B.Cu) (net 26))
 (segment (start 192.151 106.172) (end 191.389 105.41) (width 0.1524) (layer B.Cu) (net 26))
 (segment (start 191.389 105.41) (end 191.389 102.87) (width 0.1524) (layer B.Cu) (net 26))
 (segment (start 191.389 102.87) (end 190.119 101.6) (width 0.1524) (layer B.Cu) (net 26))
 (segment (start 190.119 101.6) (end 190.119 101.981) (width 0.1524) (layer B.Cu) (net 26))
 (segment (start 193.234 109.72) (end 192.5995 109.72) (width 0.1524) (layer F.Cu) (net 4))
 (segment (start 192.5995 109.72) (end 191.9485 110.371) (width 0.1524) (layer F.Cu) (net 4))
 (segment (start 193.234 108.72) (end 191.889 108.72) (width 0.1524) (layer F.Cu) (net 2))
 (segment (start 190.9485 109.6605) (end 190.9485 110.371) (width 0.1524) (layer F.Cu) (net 2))
 (segment (start 191.889 108.72) (end 190.9485 109.6605) (width 0.1524) (layer F.Cu) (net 2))
 (segment (start 193.234 109.22) (end 192.024 109.22) (width 0.1524) (layer F.Cu) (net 3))
 (segment (start 191.4485 109.7955) (end 191.4485 110.371) (width 0.1524) (layer F.Cu) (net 3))
 (segment (start 192.024 109.22) (end 191.4485 109.7955) (width 0.1524) (layer F.Cu) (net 3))
 (segment (start 193.234 108.22) (end 191.8175 108.22) (width 0.1524) (layer F.Cu) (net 1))
 (segment (start 190.4485 109.589) (end 190.4485 110.371) (width 0.1524) (layer F.Cu) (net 1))
 (segment (start 191.8175 108.22) (end 190.4485 109.589) (width 0.1524) (layer F.Cu) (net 1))
 (segment (start 197.164 108.22) (end 198.5525 108.22) (width 0.1524) (layer F.Cu) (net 15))
 (segment (start 198.5525 108.22) (end 198.5765 108.196) (width 0.1524) (layer F.Cu) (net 15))
 (segment (start 197.164 108.22) (end 197.215 108.22) (width 0.1524) (layer F.Cu) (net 15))
 (segment (start 197.164 110.22) (end 197.205802 110.22) (width 0.1524) (layer F.Cu) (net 11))
 (segment (start 197.205802 110.22) (end 197.866 110.880198) (width 0.1524) (layer F.Cu) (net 11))
 (segment (start 199.5765 108.5175) (end 199.5765 108.196) (width 0.1524) (layer F.Cu) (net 11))
 (segment (start 199.771698 108.712698) (end 199.5765 108.5175) (width 0.1524) (layer F.Cu) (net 11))
 (segment (start 199.771698 110.0455) (end 199.771698 108.712698) (width 0.1524) (layer F.Cu) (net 11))
 (segment (start 198.937 110.880198) (end 199.771698 110.0455) (width 0.1524) (layer F.Cu) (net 11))
 (segment (start 197.866 110.880198) (end 198.937 110.880198) (width 0.1524) (layer F.Cu) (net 11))
 (segment (start 197.164 110.22) (end 197.215 110.22) (width 0.1524) (layer F.Cu) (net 11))
 (segment (start 197.164 109.22) (end 197.6755 109.22) (width 0.1524) (layer F.Cu) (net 13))
 (segment (start 199.0765 109.1525) (end 199.0765 108.196) (width 0.1524) (layer F.Cu) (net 13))
 (segment (start 198.628 109.601) (end 199.0765 109.1525) (width 0.1524) (layer F.Cu) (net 13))
 (segment (start 198.0565 109.601) (end 198.628 109.601) (width 0.1524) (layer F.Cu) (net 13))
 (segment (start 197.6755 109.22) (end 198.0565 109.601) (width 0.1524) (layer F.Cu) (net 13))
 (segment (start 196.199 111.185) (end 199.076 111.185) (width 0.1524) (layer F.Cu) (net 10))
 (segment (start 200.0765 110.1845) (end 200.0765 108.196) (width 0.1524) (layer F.Cu) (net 10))
 (segment (start 199.076 111.185) (end 200.0765 110.1845) (width 0.1524) (layer F.Cu) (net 10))
 (segment (start 197.164 109.72) (end 197.731 109.72) (width 0.1524) (layer F.Cu) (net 12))
 (segment (start 198.247 110.236) (end 199.8345 111.8235) (width 0.1524) (layer B.Cu) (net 12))
 (via (at 198.247 110.236) (size 0.65) (drill 0.5) (layers F.Cu B.Cu) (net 12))
 (segment (start 197.731 109.72) (end 198.247 110.236) (width 0.1524) (layer F.Cu) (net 12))
 (segment (start 199.8345 111.8235) (end 200.279 111.8235) (width 0.1524) (layer B.Cu) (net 12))
 (segment (start 194.5005 111.3575) (end 194.5005 112.3315) (width 0.1524) (layer B.Cu) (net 7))
 (segment (start 194.699 112.133) (end 194.5005 112.3315) (width 0.1524) (layer F.Cu) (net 7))
 (via (at 194.5005 112.3315) (size 0.65) (drill 0.5) (layers F.Cu B.Cu) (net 7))
 (segment (start 194.699 112.133) (end 194.699 111.185) (width 0.1524) (layer F.Cu) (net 7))
 (segment (start 194.5005 111.3575) (end 194.3315 111.1885) (width 0.1524) (layer B.Cu) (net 7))
 (segment (start 195.199 116.84) (end 195.326 116.84) (width 0.1524) (layer F.Cu) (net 29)))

